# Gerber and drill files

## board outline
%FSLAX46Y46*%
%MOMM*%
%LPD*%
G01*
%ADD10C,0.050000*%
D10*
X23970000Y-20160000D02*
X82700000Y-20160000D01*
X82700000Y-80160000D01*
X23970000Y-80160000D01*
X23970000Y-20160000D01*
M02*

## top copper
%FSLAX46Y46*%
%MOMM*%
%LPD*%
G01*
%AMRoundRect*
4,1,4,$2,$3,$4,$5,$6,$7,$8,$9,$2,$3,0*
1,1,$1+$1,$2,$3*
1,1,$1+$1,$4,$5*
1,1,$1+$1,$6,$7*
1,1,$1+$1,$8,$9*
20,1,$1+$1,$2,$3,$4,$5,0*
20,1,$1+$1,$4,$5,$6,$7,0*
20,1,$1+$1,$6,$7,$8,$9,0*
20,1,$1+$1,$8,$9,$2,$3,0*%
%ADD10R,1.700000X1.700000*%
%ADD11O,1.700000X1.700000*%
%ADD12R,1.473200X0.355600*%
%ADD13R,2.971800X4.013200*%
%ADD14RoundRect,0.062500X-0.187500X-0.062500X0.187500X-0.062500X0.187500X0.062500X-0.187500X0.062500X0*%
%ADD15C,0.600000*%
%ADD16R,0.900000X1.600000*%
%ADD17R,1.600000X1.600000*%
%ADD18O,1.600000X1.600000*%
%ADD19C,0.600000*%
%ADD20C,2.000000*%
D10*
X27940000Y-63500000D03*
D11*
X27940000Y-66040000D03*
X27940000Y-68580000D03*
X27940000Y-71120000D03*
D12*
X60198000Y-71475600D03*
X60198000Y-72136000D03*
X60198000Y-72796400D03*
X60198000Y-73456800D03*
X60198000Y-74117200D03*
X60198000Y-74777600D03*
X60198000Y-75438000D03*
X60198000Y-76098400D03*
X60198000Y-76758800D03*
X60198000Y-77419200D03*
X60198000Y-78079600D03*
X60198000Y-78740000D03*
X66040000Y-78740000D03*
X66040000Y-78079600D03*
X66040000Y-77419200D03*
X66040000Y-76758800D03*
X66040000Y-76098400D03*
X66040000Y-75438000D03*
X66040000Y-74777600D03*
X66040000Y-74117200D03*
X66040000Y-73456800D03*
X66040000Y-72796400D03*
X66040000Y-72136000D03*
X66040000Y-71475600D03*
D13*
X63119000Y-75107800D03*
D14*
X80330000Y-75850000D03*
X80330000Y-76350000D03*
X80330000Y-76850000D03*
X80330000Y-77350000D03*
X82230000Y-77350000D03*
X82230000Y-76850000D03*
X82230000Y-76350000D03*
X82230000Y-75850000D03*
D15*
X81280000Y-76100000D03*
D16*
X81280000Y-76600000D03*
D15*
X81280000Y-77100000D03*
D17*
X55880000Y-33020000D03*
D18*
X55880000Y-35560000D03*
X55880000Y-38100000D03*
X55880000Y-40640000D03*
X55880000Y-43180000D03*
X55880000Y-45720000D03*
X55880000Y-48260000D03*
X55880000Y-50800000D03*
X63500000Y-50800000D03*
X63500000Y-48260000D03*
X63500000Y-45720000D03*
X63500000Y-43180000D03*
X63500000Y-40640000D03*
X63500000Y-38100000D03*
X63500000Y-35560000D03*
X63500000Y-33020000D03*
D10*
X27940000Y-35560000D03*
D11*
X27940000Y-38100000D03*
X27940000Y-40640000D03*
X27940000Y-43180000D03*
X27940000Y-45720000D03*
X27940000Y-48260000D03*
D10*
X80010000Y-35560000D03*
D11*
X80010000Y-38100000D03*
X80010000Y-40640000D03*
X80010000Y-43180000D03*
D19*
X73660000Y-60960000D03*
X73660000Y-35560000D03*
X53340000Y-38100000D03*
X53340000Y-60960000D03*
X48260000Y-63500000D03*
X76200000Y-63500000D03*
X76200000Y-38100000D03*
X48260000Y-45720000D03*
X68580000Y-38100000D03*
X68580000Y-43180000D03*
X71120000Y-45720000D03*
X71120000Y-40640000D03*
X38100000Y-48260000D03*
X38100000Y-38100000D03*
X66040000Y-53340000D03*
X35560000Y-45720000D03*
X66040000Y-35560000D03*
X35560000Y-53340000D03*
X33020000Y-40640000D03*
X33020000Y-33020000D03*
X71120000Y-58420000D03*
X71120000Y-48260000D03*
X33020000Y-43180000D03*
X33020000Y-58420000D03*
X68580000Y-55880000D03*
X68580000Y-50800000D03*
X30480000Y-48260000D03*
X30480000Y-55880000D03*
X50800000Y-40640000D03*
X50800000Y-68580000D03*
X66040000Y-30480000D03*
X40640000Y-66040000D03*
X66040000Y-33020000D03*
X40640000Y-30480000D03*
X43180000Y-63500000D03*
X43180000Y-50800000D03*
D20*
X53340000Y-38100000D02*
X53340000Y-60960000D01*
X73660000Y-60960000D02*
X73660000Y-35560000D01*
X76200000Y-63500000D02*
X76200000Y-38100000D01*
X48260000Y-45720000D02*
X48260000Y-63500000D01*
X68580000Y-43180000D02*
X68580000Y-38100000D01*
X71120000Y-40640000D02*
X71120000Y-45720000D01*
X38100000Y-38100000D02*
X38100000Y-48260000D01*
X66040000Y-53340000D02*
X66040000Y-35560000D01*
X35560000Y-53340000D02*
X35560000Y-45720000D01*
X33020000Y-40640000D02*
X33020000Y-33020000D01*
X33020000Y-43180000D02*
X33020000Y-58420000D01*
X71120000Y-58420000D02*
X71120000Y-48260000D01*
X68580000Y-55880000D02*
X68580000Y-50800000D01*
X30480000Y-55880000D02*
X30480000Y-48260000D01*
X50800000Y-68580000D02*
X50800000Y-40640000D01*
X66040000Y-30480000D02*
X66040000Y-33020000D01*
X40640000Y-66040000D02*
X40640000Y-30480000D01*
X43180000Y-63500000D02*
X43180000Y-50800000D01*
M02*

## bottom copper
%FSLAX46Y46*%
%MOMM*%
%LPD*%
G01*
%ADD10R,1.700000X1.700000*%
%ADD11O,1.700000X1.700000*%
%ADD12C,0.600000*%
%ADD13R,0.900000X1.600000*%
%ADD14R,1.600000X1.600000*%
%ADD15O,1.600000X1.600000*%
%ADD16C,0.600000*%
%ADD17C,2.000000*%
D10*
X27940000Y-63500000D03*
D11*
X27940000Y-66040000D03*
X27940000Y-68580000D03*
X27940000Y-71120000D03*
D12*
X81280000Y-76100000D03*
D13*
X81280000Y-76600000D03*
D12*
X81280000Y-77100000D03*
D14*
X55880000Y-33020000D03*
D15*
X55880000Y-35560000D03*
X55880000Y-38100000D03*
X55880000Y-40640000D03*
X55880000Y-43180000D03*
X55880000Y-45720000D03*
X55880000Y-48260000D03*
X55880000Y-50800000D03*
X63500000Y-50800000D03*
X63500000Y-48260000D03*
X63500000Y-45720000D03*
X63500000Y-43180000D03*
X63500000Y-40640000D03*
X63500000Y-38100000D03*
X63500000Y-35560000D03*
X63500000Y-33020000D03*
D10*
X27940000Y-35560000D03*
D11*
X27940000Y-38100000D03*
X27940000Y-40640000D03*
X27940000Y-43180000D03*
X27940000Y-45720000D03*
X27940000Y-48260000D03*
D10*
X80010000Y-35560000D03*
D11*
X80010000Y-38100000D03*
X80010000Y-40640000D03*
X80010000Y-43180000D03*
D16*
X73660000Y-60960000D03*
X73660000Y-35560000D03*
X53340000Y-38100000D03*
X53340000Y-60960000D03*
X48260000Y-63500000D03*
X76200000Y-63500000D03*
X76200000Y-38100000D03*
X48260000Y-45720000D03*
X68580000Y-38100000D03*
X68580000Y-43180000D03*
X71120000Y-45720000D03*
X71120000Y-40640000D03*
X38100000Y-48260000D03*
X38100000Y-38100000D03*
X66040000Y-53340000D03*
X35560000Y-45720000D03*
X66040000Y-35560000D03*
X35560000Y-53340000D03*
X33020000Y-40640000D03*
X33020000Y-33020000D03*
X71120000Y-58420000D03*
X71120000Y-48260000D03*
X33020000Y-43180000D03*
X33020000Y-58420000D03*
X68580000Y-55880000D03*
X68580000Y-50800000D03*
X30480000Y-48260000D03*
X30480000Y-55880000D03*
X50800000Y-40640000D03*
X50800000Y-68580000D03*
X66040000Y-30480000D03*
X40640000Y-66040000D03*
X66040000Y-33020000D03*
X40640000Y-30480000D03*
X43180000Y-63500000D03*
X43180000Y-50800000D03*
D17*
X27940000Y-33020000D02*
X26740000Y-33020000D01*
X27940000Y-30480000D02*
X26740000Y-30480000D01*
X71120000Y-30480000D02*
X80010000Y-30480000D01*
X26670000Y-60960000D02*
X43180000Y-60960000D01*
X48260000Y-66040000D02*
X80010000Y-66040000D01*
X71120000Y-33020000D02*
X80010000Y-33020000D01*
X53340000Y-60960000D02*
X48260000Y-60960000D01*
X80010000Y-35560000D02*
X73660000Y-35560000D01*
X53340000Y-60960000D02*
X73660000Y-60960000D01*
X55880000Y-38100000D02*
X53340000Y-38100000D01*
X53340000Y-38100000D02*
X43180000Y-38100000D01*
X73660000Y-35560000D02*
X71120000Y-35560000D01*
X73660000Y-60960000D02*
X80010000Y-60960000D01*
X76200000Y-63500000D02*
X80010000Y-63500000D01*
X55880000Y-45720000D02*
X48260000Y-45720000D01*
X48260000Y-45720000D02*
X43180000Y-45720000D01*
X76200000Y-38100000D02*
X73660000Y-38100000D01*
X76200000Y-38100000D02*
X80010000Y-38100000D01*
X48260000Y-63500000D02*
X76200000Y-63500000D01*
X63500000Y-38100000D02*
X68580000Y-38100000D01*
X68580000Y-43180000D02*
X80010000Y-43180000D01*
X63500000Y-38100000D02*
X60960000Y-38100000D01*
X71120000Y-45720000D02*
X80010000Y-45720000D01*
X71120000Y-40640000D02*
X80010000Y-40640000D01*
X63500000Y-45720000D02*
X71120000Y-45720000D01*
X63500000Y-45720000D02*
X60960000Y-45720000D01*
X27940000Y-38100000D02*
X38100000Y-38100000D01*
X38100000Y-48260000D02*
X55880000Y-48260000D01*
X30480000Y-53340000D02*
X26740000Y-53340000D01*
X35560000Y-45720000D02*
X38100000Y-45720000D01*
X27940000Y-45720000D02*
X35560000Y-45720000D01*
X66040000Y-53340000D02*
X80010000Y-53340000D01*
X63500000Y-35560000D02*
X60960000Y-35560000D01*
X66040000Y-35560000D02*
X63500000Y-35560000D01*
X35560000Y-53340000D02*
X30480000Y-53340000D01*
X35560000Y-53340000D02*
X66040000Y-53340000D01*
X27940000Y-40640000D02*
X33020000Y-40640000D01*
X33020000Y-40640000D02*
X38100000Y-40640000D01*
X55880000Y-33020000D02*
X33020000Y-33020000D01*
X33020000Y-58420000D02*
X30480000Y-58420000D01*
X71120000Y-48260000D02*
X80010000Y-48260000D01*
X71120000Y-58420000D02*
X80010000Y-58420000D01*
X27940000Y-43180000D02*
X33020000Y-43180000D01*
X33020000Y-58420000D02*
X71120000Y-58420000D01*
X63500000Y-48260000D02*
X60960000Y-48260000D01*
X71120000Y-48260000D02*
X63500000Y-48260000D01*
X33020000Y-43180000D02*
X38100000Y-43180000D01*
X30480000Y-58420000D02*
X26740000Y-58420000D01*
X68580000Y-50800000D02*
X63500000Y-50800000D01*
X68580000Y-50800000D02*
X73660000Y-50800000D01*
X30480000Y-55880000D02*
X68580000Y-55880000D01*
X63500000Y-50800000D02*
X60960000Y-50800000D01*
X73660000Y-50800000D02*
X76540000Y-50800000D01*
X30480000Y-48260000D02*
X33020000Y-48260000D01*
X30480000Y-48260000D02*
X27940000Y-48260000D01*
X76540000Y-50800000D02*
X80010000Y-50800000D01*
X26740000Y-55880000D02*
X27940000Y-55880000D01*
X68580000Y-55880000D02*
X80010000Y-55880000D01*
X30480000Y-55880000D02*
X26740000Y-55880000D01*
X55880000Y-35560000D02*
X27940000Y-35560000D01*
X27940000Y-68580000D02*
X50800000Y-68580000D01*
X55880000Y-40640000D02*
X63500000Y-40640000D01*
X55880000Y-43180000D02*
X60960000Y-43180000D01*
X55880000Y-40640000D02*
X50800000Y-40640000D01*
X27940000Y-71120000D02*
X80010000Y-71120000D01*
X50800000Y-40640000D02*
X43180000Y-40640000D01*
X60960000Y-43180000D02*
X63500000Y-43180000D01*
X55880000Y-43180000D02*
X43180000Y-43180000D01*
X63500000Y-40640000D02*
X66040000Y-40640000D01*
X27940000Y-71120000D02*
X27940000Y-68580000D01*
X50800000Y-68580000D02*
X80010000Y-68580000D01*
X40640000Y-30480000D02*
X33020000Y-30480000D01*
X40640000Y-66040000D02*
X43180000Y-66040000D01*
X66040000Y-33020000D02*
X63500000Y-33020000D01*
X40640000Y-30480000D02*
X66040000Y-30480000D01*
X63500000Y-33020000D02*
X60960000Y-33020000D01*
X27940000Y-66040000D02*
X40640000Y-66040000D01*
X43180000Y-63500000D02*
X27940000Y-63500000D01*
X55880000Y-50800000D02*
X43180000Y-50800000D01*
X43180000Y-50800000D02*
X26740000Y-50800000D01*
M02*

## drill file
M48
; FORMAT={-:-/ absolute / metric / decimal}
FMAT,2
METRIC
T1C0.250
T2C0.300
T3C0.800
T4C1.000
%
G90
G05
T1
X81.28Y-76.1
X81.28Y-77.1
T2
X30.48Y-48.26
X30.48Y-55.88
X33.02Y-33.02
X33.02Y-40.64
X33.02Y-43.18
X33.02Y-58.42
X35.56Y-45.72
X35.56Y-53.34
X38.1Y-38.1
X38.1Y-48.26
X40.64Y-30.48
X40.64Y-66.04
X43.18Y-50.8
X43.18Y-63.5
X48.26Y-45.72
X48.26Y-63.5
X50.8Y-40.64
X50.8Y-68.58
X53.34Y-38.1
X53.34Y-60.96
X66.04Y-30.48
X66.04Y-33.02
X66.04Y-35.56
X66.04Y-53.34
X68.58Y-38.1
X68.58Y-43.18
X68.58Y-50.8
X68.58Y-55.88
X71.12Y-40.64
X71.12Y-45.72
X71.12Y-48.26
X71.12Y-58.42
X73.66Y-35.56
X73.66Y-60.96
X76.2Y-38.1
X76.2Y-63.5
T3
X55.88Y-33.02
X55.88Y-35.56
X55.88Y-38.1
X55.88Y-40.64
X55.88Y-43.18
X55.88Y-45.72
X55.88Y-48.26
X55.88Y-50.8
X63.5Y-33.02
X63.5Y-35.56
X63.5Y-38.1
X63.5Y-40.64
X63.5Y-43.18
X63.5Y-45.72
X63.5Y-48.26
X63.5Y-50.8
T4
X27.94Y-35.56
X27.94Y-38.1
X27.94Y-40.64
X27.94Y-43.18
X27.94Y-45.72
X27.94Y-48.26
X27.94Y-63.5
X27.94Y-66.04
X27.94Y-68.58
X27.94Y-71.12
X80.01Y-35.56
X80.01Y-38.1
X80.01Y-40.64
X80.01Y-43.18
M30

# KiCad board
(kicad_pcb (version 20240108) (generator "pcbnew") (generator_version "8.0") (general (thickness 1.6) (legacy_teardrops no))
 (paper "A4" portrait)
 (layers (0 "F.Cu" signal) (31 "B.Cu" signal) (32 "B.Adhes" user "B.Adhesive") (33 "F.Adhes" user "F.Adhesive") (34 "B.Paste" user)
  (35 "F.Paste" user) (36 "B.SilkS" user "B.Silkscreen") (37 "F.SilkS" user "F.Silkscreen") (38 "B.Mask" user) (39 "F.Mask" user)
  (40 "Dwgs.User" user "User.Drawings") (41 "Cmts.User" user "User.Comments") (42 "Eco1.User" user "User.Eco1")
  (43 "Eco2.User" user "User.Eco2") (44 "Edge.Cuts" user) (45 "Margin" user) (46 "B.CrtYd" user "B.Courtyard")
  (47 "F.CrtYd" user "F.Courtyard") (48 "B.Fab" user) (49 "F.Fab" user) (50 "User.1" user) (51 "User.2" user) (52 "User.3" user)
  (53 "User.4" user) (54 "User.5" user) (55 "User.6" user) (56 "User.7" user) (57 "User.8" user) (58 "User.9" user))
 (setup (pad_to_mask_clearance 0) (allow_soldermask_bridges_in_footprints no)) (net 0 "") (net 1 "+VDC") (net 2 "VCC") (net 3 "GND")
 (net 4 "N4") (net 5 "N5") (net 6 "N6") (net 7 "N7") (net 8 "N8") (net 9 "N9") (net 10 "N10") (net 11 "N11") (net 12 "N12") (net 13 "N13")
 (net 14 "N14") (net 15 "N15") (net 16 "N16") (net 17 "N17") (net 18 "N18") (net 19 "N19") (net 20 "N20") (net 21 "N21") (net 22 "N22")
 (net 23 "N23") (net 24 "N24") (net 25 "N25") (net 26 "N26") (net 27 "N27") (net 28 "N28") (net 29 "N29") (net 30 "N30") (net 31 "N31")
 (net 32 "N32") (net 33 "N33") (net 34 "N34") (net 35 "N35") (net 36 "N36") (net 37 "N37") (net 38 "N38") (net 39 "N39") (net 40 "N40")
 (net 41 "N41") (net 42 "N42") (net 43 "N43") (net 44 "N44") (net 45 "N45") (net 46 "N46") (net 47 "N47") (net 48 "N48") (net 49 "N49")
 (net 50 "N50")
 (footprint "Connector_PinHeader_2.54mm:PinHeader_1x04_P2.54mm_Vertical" (layer "F.Cu") (at 27.94 63.5)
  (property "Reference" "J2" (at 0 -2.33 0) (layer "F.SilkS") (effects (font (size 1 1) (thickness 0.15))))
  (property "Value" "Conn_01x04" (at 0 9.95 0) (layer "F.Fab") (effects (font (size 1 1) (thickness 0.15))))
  (pad "1" thru_hole rect (at 0 0) (size 1.7 1.7) (drill 1) (layers "*.Cu" "*.Mask") (remove_unused_layers no) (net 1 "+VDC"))
  (pad "2" thru_hole oval (at 0 2.54) (size 1.7 1.7) (drill 1) (layers "*.Cu" "*.Mask") (remove_unused_layers no) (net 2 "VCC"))
  (pad "3" thru_hole oval (at 0 5.08) (size 1.7 1.7) (drill 1) (layers "*.Cu" "*.Mask") (remove_unused_layers no) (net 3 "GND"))
  (pad "4" thru_hole oval (at 0 7.62) (size 1.7 1.7) (drill 1) (layers "*.Cu" "*.Mask") (remove_unused_layers no) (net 3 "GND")))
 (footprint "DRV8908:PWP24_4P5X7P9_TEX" (layer "F.Cu") (at 63.119 75.1078)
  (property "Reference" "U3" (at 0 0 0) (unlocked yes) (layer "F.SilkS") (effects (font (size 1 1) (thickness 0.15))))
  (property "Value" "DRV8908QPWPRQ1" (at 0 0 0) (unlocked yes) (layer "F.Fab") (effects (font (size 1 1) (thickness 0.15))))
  (pad "1" smd rect (at -2.921 -3.6322) (size 1.4732 0.3556) (layers "F.Cu" "F.Paste" "F.Mask") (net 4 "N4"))
  (pad "2" smd rect (at -2.921 -2.9718) (size 1.4732 0.3556) (layers "F.Cu" "F.Paste" "F.Mask") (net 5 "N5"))
  (pad "3" smd rect (at -2.921 -2.3114) (size 1.4732 0.3556) (layers "F.Cu" "F.Paste" "F.Mask") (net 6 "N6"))
  (pad "4" smd rect (at -2.921 -1.651) (size 1.4732 0.3556) (layers "F.Cu" "F.Paste" "F.Mask") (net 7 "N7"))
  (pad "5" smd rect (at -2.921 -0.9906) (size 1.4732 0.3556) (layers "F.Cu" "F.Paste" "F.Mask") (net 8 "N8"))
  (pad "6" smd rect (at -2.921 -0.3302) (size 1.4732 0.3556) (layers "F.Cu" "F.Paste" "F.Mask") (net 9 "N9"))
  (pad "7" smd rect (at -2.921 0.3302) (size 1.4732 0.3556) (layers "F.Cu" "F.Paste" "F.Mask") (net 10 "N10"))
  (pad "8" smd rect (at -2.921 0.9906) (size 1.4732 0.3556) (layers "F.Cu" "F.Paste" "F.Mask") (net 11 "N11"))
  (pad "9" smd rect (at -2.921 1.651) (size 1.4732 0.3556) (layers "F.Cu" "F.Paste" "F.Mask") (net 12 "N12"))
  (pad "10" smd rect (at -2.921 2.3114) (size 1.4732 0.3556) (layers "F.Cu" "F.Paste" "F.Mask") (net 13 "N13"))
  (pad "11" smd rect (at -2.921 2.9718) (size 1.4732 0.3556) (layers "F.Cu" "F.Paste" "F.Mask") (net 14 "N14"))
  (pad "12" smd rect (at -2.921 3.6322) (size 1.4732 0.3556) (layers "F.Cu" "F.Paste" "F.Mask") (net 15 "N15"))
  (pad "13" smd rect (at 2.921 3.6322) (size 1.4732 0.3556) (layers "F.Cu" "F.Paste" "F.Mask") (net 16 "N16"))
  (pad "14" smd rect (at 2.921 2.9718) (size 1.4732 0.3556) (layers "F.Cu" "F.Paste" "F.Mask") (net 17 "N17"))
  (pad "15" smd rect (at 2.921 2.3114) (size 1.4732 0.3556) (layers "F.Cu" "F.Paste" "F.Mask") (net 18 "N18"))
  (pad "16" smd rect (at 2.921 1.651) (size 1.4732 0.3556) (layers "F.Cu" "F.Paste" "F.Mask") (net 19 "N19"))
  (pad "17" smd rect (at 2.921 0.9906) (size 1.4732 0.3556) (layers "F.Cu" "F.Paste" "F.Mask") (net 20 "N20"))
  (pad "18" smd rect (at 2.921 0.3302) (size 1.4732 0.3556) (layers "F.Cu" "F.Paste" "F.Mask") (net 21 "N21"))
  (pad "19" smd rect (at 2.921 -0.3302) (size 1.4732 0.3556) (layers "F.Cu" "F.Paste" "F.Mask") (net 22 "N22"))
  (pad "20" smd rect (at 2.921 -0.9906) (size 1.4732 0.3556) (layers "F.Cu" "F.Paste" "F.Mask") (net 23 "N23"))
  (pad "21" smd rect (at 2.921 -1.651) (size 1.4732 0.3556) (layers "F.Cu" "F.Paste" "F.Mask") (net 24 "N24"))
  (pad "22" smd rect (at 2.921 -2.3114) (size 1.4732 0.3556) (layers "F.Cu" "F.Paste" "F.Mask") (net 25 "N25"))
  (pad "23" smd rect (at 2.921 -2.9718) (size 1.4732 0.3556) (layers "F.Cu" "F.Paste" "F.Mask") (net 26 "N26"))
  (pad "24" smd rect (at 2.921 -3.6322) (size 1.4732 0.3556) (layers "F.Cu" "F.Paste" "F.Mask") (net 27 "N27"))
  (pad "EPAD" smd rect (at 0 0) (size 2.9718 4.0132) (layers "F.Cu" "F.Mask") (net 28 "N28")))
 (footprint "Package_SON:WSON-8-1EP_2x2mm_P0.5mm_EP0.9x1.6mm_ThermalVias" (layer "F.Cu") (at 81.28 76.6)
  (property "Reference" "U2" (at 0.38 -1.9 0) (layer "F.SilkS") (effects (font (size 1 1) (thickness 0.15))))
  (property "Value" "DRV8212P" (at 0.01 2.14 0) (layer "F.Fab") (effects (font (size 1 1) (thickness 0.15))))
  (pad "" smd rect (at 0 -0.4) (size 0.75 0.65) (layers "F.Paste"))
  (pad "" smd rect (at 0 0.4) (size 0.75 0.65) (layers "F.Paste"))
  (pad "1" smd roundrect (at -0.95 -0.75) (size 0.5 0.25) (layers "F.Cu" "F.Paste" "F.Mask") (roundrect_rratio 0.25) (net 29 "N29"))
  (pad "2" smd roundrect (at -0.95 -0.25) (size 0.5 0.25) (layers "F.Cu" "F.Paste" "F.Mask") (roundrect_rratio 0.25) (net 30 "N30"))
  (pad "3" smd roundrect (at -0.95 0.25) (size 0.5 0.25) (layers "F.Cu" "F.Paste" "F.Mask") (roundrect_rratio 0.25) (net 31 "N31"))
  (pad "4" smd roundrect (at -0.95 0.75) (size 0.5 0.25) (layers "F.Cu" "F.Paste" "F.Mask") (roundrect_rratio 0.25) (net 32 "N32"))
  (pad "5" smd roundrect (at 0.95 0.75) (size 0.5 0.25) (layers "F.Cu" "F.Paste" "F.Mask") (roundrect_rratio 0.25) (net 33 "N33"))
  (pad "6" smd roundrect (at 0.95 0.25) (size 0.5 0.25) (layers "F.Cu" "F.Paste" "F.Mask") (roundrect_rratio 0.25) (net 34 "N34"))
  (pad "7" smd roundrect (at 0.95 -0.25) (size 0.5 0.25) (layers "F.Cu" "F.Paste" "F.Mask") (roundrect_rratio 0.25) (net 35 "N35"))
  (pad "8" smd roundrect (at 0.95 -0.75) (size 0.5 0.25) (layers "F.Cu" "F.Paste" "F.Mask") (roundrect_rratio 0.25) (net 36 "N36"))
  (pad "9" thru_hole circle (at 0 -0.5) (size 0.6 0.6) (drill 0.25) (layers "*.Cu") (remove_unused_layers no) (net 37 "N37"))
  (pad "9" smd rect (at 0 0) (size 0.9 1.6) (layers "F.Cu" "F.Mask") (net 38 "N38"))
  (pad "9" smd rect (at 0 0) (size 0.9 1.6) (layers "B.Cu") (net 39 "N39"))
  (pad "9" thru_hole circle (at 0 0.5) (size 0.6 0.6) (drill 0.25) (layers "*.Cu") (remove_unused_layers no) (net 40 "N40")))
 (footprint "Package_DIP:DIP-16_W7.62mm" (layer "F.Cu") (at 55.88 33.02)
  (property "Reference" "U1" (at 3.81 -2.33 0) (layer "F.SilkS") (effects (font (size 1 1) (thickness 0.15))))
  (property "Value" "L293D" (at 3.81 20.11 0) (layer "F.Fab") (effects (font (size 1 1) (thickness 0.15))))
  (pad "1" thru_hole rect (at 0 0) (size 1.6 1.6) (drill 0.8) (layers "*.Cu" "*.Mask") (remove_unused_layers no) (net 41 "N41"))
  (pad "2" thru_hole oval (at 0 2.54) (size 1.6 1.6) (drill 0.8) (layers "*.Cu" "*.Mask") (remove_unused_layers no) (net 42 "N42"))
  (pad "3" thru_hole oval (at 0 5.08) (size 1.6 1.6) (drill 0.8) (layers "*.Cu" "*.Mask") (remove_unused_layers no) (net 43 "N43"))
  (pad "4" thru_hole oval (at 0 7.62) (size 1.6 1.6) (drill 0.8) (layers "*.Cu" "*.Mask") (remove_unused_layers no) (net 3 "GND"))
  (pad "5" thru_hole oval (at 0 10.16) (size 1.6 1.6) (drill 0.8) (layers "*.Cu" "*.Mask") (remove_unused_layers no) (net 3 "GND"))
  (pad "6" thru_hole oval (at 0 12.7) (size 1.6 1.6) (drill 0.8) (layers "*.Cu" "*.Mask") (remove_unused_layers no) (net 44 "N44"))
  (pad "7" thru_hole oval (at 0 15.24) (size 1.6 1.6) (drill 0.8) (layers "*.Cu" "*.Mask") (remove_unused_layers no) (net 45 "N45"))
  (pad "8" thru_hole oval (at 0 17.78) (size 1.6 1.6) (drill 0.8) (layers "*.Cu" "*.Mask") (remove_unused_layers no) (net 1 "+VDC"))
  (pad "9" thru_hole oval (at 7.62 17.78) (size 1.6 1.6) (drill 0.8) (layers "*.Cu" "*.Mask") (remove_unused_layers no) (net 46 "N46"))
  (pad "10" thru_hole oval (at 7.62 15.24) (size 1.6 1.6) (drill 0.8) (layers "*.Cu" "*.Mask") (remove_unused_layers no) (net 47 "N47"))
  (pad "11" thru_hole oval (at 7.62 12.7) (size 1.6 1.6) (drill 0.8) (layers "*.Cu" "*.Mask") (remove_unused_layers no) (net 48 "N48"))
  (pad "12" thru_hole oval (at 7.62 10.16) (size 1.6 1.6) (drill 0.8) (layers "*.Cu" "*.Mask") (remove_unused_layers no) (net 3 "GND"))
  (pad "13" thru_hole oval (at 7.62 7.62) (size 1.6 1.6) (drill 0.8) (layers "*.Cu" "*.Mask") (remove_unused_layers no) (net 3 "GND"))
  (pad "14" thru_hole oval (at 7.62 5.08) (size 1.6 1.6) (drill 0.8) (layers "*.Cu" "*.Mask") (remove_unused_layers no) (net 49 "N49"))
  (pad "15" thru_hole oval (at 7.62 2.54) (size 1.6 1.6) (drill 0.8) (layers "*.Cu" "*.Mask") (remove_unused_layers no) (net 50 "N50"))
  (pad "16" thru_hole oval (at 7.62 0) (size 1.6 1.6) (drill 0.8) (layers "*.Cu" "*.Mask") (remove_unused_layers no) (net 2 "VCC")))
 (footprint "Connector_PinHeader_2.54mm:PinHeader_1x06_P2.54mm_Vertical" (layer "F.Cu") (at 27.94 35.56)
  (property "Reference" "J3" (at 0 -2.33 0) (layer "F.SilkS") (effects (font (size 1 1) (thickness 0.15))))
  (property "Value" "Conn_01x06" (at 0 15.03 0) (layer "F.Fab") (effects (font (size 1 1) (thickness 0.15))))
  (pad "1" thru_hole rect (at 0 0) (size 1.7 1.7) (drill 1) (layers "*.Cu" "*.Mask") (remove_unused_layers no) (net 42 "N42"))
  (pad "2" thru_hole oval (at 0 2.54) (size 1.7 1.7) (drill 1) (layers "*.Cu" "*.Mask") (remove_unused_layers no) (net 45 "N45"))
  (pad "3" thru_hole oval (at 0 5.08) (size 1.7 1.7) (drill 1) (layers "*.Cu" "*.Mask") (remove_unused_layers no) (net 41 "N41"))
  (pad "4" thru_hole oval (at 0 7.62) (size 1.7 1.7) (drill 1) (layers "*.Cu" "*.Mask") (remove_unused_layers no) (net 47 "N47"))
  (pad "5" thru_hole oval (at 0 10.16) (size 1.7 1.7) (drill 1) (layers "*.Cu" "*.Mask") (remove_unused_layers no) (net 50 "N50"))
  (pad "6" thru_hole oval (at 0 12.7) (size 1.7 1.7) (drill 1) (layers "*.Cu" "*.Mask") (remove_unused_layers no) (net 46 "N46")))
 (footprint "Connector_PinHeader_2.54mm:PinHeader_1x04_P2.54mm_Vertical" (layer "F.Cu") (at 80.01 35.56)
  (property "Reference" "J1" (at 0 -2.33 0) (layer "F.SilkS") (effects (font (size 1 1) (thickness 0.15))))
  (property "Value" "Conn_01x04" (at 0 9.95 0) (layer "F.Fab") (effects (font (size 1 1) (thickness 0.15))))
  (pad "1" thru_hole rect (at 0 0) (size 1.7 1.7) (drill 1) (layers "*.Cu" "*.Mask") (remove_unused_layers no) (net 43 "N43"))
  (pad "2" thru_hole oval (at 0 2.54) (size 1.7 1.7) (drill 1) (layers "*.Cu" "*.Mask") (remove_unused_layers no) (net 44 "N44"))
  (pad "3" thru_hole oval (at 0 5.08) (size 1.7 1.7) (drill 1) (layers "*.Cu" "*.Mask") (remove_unused_layers no) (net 48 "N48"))
  (pad "4" thru_hole oval (at 0 7.62) (size 1.7 1.7) (drill 1) (layers "*.Cu" "*.Mask") (remove_unused_layers no) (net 49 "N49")))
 (gr_rect (start 23.97 20.16) (end 82.7 80.16) (stroke (width 0.05) (type default)) (fill none) (layer "Edge.Cuts"))
 (segment (start 27.94 33.02) (end 26.74 33.02) (width 2) (layer "B.Cu") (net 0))
 (segment (start 27.94 30.48) (end 26.74 30.48) (width 2) (layer "B.Cu") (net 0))
 (segment (start 71.12 30.48) (end 80.01 30.48) (width 2) (layer "B.Cu") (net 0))
 (segment (start 26.67 60.96) (end 43.18 60.96) (width 2) (layer "B.Cu") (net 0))
 (segment (start 48.26 66.04) (end 80.01 66.04) (width 2) (layer "B.Cu") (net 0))
 (segment (start 71.12 33.02) (end 80.01 33.02) (width 2) (layer "B.Cu") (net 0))
 (segment (start 53.34 38.1) (end 53.34 60.96) (width 2) (layer "F.Cu") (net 43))
 (segment (start 73.66 60.96) (end 73.66 35.56) (width 2) (layer "F.Cu") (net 43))
 (via (at 73.66 60.96) (size 0.6) (drill 0.3) (layers "F.Cu" "B.Cu") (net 43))
 (via (at 73.66 35.56) (size 0.6) (drill 0.3) (layers "F.Cu" "B.Cu") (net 43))
 (via (at 53.34 38.1) (size 0.6) (drill 0.3) (layers "F.Cu" "B.Cu") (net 43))
 (via (at 53.34 60.96) (size 0.6) (drill 0.3) (layers "F.Cu" "B.Cu") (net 43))
 (segment (start 53.34 60.96) (end 48.26 60.96) (width 2) (layer "B.Cu") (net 43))
 (segment (start 80.01 35.56) (end 73.66 35.56) (width 2) (layer "B.Cu") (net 43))
 (segment (start 53.34 60.96) (end 73.66 60.96) (width 2) (layer "B.Cu") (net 43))
 (segment (start 55.88 38.1) (end 53.34 38.1) (width 2) (layer "B.Cu") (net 43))
 (segment (start 53.34 38.1) (end 43.18 38.1) (width 2) (layer "B.Cu") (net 43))
 (segment (start 73.66 35.56) (end 71.12 35.56) (width 2) (layer "B.Cu") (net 43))
 (segment (start 73.66 60.96) (end 80.01 60.96) (width 2) (layer "B.Cu") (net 43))
 (segment (start 76.2 63.5) (end 76.2 38.1) (width 2) (layer "F.Cu") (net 44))
 (segment (start 48.26 45.72) (end 48.26 63.5) (width 2) (layer "F.Cu") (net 44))
 (via (at 48.26 63.5) (size 0.6) (drill 0.3) (layers "F.Cu" "B.Cu") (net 44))
 (via (at 76.2 63.5) (size 0.6) (drill 0.3) (layers "F.Cu" "B.Cu") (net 44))
 (via (at 76.2 38.1) (size 0.6) (drill 0.3) (layers "F.Cu" "B.Cu") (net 44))
 (via (at 48.26 45.72) (size 0.6) (drill 0.3) (layers "F.Cu" "B.Cu") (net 44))
 (segment (start 76.2 63.5) (end 80.01 63.5) (width 2) (layer "B.Cu") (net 44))
 (segment (start 55.88 45.72) (end 48.26 45.72) (width 2) (layer "B.Cu") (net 44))
 (segment (start 48.26 45.72) (end 43.18 45.72) (width 2) (layer "B.Cu") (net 44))
 (segment (start 76.2 38.1) (end 73.66 38.1) (width 2) (layer "B.Cu") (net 44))
 (segment (start 76.2 38.1) (end 80.01 38.1) (width 2) (layer "B.Cu") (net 44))
 (segment (start 48.26 63.5) (end 76.2 63.5) (width 2) (layer "B.Cu") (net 44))
 (segment (start 68.58 43.18) (end 68.58 38.1) (width 2) (layer "F.Cu") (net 49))
 (via (at 68.58 38.1) (size 0.6) (drill 0.3) (layers "F.Cu" "B.Cu") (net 49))
 (via (at 68.58 43.18) (size 0.6) (drill 0.3) (layers "F.Cu" "B.Cu") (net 49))
 (segment (start 63.5 38.1) (end 68.58 38.1) (width 2) (layer "B.Cu") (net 49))
 (segment (start 68.58 43.18) (end 80.01 43.18) (width 2) (layer "B.Cu") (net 49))
 (segment (start 63.5 38.1) (end 60.96 38.1) (width 2) (layer "B.Cu") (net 49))
 (segment (start 71.12 40.64) (end 71.12 45.72) (width 2) (layer "F.Cu") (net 48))
 (via (at 71.12 45.72) (size 0.6) (drill 0.3) (layers "F.Cu" "B.Cu") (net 48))
 (via (at 71.12 40.64) (size 0.6) (drill 0.3) (layers "F.Cu" "B.Cu") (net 48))
 (segment (start 71.12 45.72) (end 80.01 45.72) (width 2) (layer "B.Cu") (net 48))
 (segment (start 71.12 40.64) (end 80.01 40.64) (width 2) (layer "B.Cu") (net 48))
 (segment (start 63.5 45.72) (end 71.12 45.72) (width 2) (layer "B.Cu") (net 48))
 (segment (start 63.5 45.72) (end 60.96 45.72) (width 2) (layer "B.Cu") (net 48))
 (segment (start 38.1 38.1) (end 38.1 48.26) (width 2) (layer "F.Cu") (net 45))
 (via (at 38.1 48.26) (size 0.6) (drill 0.3) (layers "F.Cu" "B.Cu") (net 45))
 (via (at 38.1 38.1) (size 0.6) (drill 0.3) (layers "F.Cu" "B.Cu") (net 45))
 (segment (start 27.94 38.1) (end 38.1 38.1) (width 2) (layer "B.Cu") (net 45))
 (segment (start 38.1 48.26) (end 55.88 48.26) (width 2) (layer "B.Cu") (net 45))
 (segment (start 66.04 53.34) (end 66.04 35.56) (width 2) (layer "F.Cu") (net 50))
 (segment (start 35.56 53.34) (end 35.56 45.72) (width 2) (layer "F.Cu") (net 50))
 (via (at 66.04 53.34) (size 0.6) (drill 0.3) (layers "F.Cu" "B.Cu") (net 50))
 (via (at 35.56 45.72) (size 0.6) (drill 0.3) (layers "F.Cu" "B.Cu") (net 50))
 (via (at 66.04 35.56) (size 0.6) (drill 0.3) (layers "F.Cu" "B.Cu") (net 50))
 (via (at 35.56 53.34) (size 0.6) (drill 0.3) (layers "F.Cu" "B.Cu") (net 50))
 (segment (start 30.48 53.34) (end 26.74 53.34) (width 2) (layer "B.Cu") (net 50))
 (segment (start 35.56 45.72) (end 38.1 45.72) (width 2) (layer "B.Cu") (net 50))
 (segment (start 27.94 45.72) (end 35.56 45.72) (width 2) (layer "B.Cu") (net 50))
 (segment (start 66.04 53.34) (end 80.01 53.34) (width 2) (layer "B.Cu") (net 50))
 (segment (start 63.5 35.56) (end 60.96 35.56) (width 2) (layer "B.Cu") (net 50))
 (segment (start 66.04 35.56) (end 63.5 35.56) (width 2) (layer "B.Cu") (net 50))
 (segment (start 35.56 53.34) (end 30.48 53.34) (width 2) (layer "B.Cu") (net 50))
 (segment (start 35.56 53.34) (end 66.04 53.34) (width 2) (layer "B.Cu") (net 50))
 (segment (start 33.02 40.64) (end 33.02 33.02) (width 2) (layer "F.Cu") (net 41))
 (via (at 33.02 40.64) (size 0.6) (drill 0.3) (layers "F.Cu" "B.Cu") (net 41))
 (via (at 33.02 33.02) (size 0.6) (drill 0.3) (layers "F.Cu" "B.Cu") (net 41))
 (segment (start 27.94 40.64) (end 33.02 40.64) (width 2) (layer "B.Cu") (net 41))
 (segment (start 33.02 40.64) (end 38.1 40.64) (width 2) (layer "B.Cu") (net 41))
 (segment (start 55.88 33.02) (end 33.02 33.02) (width 2) (layer "B.Cu") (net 41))
 (segment (start 33.02 43.18) (end 33.02 58.42) (width 2) (layer "F.Cu") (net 47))
 (segment (start 71.12 58.42) (end 71.12 48.26) (width 2) (layer "F.Cu") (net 47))
 (via (at 71.12 58.42) (size 0.6) (drill 0.3) (layers "F.Cu" "B.Cu") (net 47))
 (via (at 71.12 48.26) (size 0.6) (drill 0.3) (layers "F.Cu" "B.Cu") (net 47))
 (via (at 33.02 43.18) (size 0.6) (drill 0.3) (layers "F.Cu" "B.Cu") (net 47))
 (via (at 33.02 58.42) (size 0.6) (drill 0.3) (layers "F.Cu" "B.Cu") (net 47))
 (segment (start 33.02 58.42) (end 30.48 58.42) (width 2) (layer "B.Cu") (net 47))
 (segment (start 71.12 48.26) (end 80.01 48.26) (width 2) (layer "B.Cu") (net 47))
 (segment (start 71.12 58.42) (end 80.01 58.42) (width 2) (layer "B.Cu") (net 47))
 (segment (start 27.94 43.18) (end 33.02 43.18) (width 2) (layer "B.Cu") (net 47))
 (segment (start 33.02 58.42) (end 71.12 58.42) (width 2) (layer "B.Cu") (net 47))
 (segment (start 63.5 48.26) (end 60.96 48.26) (width 2) (layer "B.Cu") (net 47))
 (segment (start 71.12 48.26) (end 63.5 48.26) (width 2) (layer "B.Cu") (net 47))
 (segment (start 33.02 43.18) (end 38.1 43.18) (width 2) (layer "B.Cu") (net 47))
 (segment (start 30.48 58.42) (end 26.74 58.42) (width 2) (layer "B.Cu") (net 47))
 (segment (start 68.58 55.88) (end 68.58 50.8) (width 2) (layer "F.Cu") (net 46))
 (segment (start 30.48 55.88) (end 30.48 48.26) (width 2) (layer "F.Cu") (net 46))
 (via (at 68.58 55.88) (size 0.6) (drill 0.3) (layers "F.Cu" "B.Cu") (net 46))
 (via (at 68.58 50.8) (size 0.6) (drill 0.3) (layers "F.Cu" "B.Cu") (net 46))
 (via (at 30.48 48.26) (size 0.6) (drill 0.3) (layers "F.Cu" "B.Cu") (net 46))
 (via (at 30.48 55.88) (size 0.6) (drill 0.3) (layers "F.Cu" "B.Cu") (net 46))
 (segment (start 68.58 50.8) (end 63.5 50.8) (width 2) (layer "B.Cu") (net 46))
 (segment (start 68.58 50.8) (end 73.66 50.8) (width 2) (layer "B.Cu") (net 46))
 (segment (start 30.48 55.88) (end 68.58 55.88) (width 2) (layer "B.Cu") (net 46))
 (segment (start 63.5 50.8) (end 60.96 50.8) (width 2) (layer "B.Cu") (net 46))
 (segment (start 73.66 50.8) (end 76.54 50.8) (width 2) (layer "B.Cu") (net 46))
 (segment (start 30.48 48.26) (end 33.02 48.26) (width 2) (layer "B.Cu") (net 46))
 (segment (start 30.48 48.26) (end 27.94 48.26) (width 2) (layer "B.Cu") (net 46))
 (segment (start 76.54 50.8) (end 80.01 50.8) (width 2) (layer "B.Cu") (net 46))
 (segment (start 26.74 55.88) (end 27.94 55.88) (width 2) (layer "B.Cu") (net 46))
 (segment (start 68.58 55.88) (end 80.01 55.88) (width 2) (layer "B.Cu") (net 46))
 (segment (start 30.48 55.88) (end 26.74 55.88) (width 2) (layer "B.Cu") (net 46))
 (segment (start 55.88 35.56) (end 27.94 35.56) (width 2) (layer "B.Cu") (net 42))
 (segment (start 50.8 68.58) (end 50.8 40.64) (width 2) (layer "F.Cu") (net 3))
 (via (at 50.8 40.64) (size 0.6) (drill 0.3) (layers "F.Cu" "B.Cu") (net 3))
 (via (at 50.8 68.58) (size 0.6) (drill 0.3) (layers "F.Cu" "B.Cu") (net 3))
 (segment (start 27.94 68.58) (end 50.8 68.58) (width 2) (layer "B.Cu") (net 3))
 (segment (start 55.88 40.64) (end 63.5 40.64) (width 2) (layer "B.Cu") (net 3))
 (segment (start 55.88 43.18) (end 60.96 43.18) (width 2) (layer "B.Cu") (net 3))
 (segment (start 55.88 40.64) (end 50.8 40.64) (width 2) (layer "B.Cu") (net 3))
 (segment (start 27.94 71.12) (end 80.01 71.12) (width 2) (layer "B.Cu") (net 3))
 (segment (start 50.8 40.64) (end 43.18 40.64) (width 2) (layer "B.Cu") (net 3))
 (segment (start 60.96 43.18) (end 63.5 43.18) (width 2) (layer "B.Cu") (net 3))
 (segment (start 55.88 43.18) (end 43.18 43.18) (width 2) (layer "B.Cu") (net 3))
 (segment (start 63.5 40.64) (end 66.04 40.64) (width 2) (layer "B.Cu") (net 3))
 (segment (start 27.94 71.12) (end 27.94 68.58) (width 2) (layer "B.Cu") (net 3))
 (segment (start 50.8 68.58) (end 80.01 68.58) (width 2) (layer "B.Cu") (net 3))
 (segment (start 66.04 30.48) (end 66.04 33.02) (width 2) (layer "F.Cu") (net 2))
 (segment (start 40.64 66.04) (end 40.64 30.48) (width 2) (layer "F.Cu") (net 2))
 (via (at 66.04 30.48) (size 0.6) (drill 0.3) (layers "F.Cu" "B.Cu") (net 2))
 (via (at 40.64 66.04) (size 0.6) (drill 0.3) (layers "F.Cu" "B.Cu") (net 2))
 (via (at 66.04 33.02) (size 0.6) (drill 0.3) (layers "F.Cu" "B.Cu") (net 2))
 (via (at 40.64 30.48) (size 0.6) (drill 0.3) (layers "F.Cu" "B.Cu") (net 2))
 (segment (start 40.64 30.48) (end 33.02 30.48) (width 2) (layer "B.Cu") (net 2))
 (segment (start 40.64 66.04) (end 43.18 66.04) (width 2) (layer "B.Cu") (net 2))
 (segment (start 66.04 33.02) (end 63.5 33.02) (width 2) (layer "B.Cu") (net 2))
 (segment (start 40.64 30.48) (end 66.04 30.48) (width 2) (layer "B.Cu") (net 2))
 (segment (start 63.5 33.02) (end 60.96 33.02) (width 2) (layer "B.Cu") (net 2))
 (segment (start 27.94 66.04) (end 40.64 66.04) (width 2) (layer "B.Cu") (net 2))
 (segment (start 43.18 63.5) (end 43.18 50.8) (width 2) (layer "F.Cu") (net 1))
 (via (at 43.18 63.5) (size 0.6) (drill 0.3) (layers "F.Cu" "B.Cu") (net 1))
 (via (at 43.18 50.8) (size 0.6) (drill 0.3) (layers "F.Cu" "B.Cu") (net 1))
 (segment (start 43.18 63.5) (end 27.94 63.5) (width 2) (layer "B.Cu") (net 1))
 (segment (start 55.88 50.8) (end 43.18 50.8) (width 2) (layer "B.Cu") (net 1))
 (segment (start 43.18 50.8) (end 26.74 50.8) (width 2) (layer "B.Cu") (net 1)))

